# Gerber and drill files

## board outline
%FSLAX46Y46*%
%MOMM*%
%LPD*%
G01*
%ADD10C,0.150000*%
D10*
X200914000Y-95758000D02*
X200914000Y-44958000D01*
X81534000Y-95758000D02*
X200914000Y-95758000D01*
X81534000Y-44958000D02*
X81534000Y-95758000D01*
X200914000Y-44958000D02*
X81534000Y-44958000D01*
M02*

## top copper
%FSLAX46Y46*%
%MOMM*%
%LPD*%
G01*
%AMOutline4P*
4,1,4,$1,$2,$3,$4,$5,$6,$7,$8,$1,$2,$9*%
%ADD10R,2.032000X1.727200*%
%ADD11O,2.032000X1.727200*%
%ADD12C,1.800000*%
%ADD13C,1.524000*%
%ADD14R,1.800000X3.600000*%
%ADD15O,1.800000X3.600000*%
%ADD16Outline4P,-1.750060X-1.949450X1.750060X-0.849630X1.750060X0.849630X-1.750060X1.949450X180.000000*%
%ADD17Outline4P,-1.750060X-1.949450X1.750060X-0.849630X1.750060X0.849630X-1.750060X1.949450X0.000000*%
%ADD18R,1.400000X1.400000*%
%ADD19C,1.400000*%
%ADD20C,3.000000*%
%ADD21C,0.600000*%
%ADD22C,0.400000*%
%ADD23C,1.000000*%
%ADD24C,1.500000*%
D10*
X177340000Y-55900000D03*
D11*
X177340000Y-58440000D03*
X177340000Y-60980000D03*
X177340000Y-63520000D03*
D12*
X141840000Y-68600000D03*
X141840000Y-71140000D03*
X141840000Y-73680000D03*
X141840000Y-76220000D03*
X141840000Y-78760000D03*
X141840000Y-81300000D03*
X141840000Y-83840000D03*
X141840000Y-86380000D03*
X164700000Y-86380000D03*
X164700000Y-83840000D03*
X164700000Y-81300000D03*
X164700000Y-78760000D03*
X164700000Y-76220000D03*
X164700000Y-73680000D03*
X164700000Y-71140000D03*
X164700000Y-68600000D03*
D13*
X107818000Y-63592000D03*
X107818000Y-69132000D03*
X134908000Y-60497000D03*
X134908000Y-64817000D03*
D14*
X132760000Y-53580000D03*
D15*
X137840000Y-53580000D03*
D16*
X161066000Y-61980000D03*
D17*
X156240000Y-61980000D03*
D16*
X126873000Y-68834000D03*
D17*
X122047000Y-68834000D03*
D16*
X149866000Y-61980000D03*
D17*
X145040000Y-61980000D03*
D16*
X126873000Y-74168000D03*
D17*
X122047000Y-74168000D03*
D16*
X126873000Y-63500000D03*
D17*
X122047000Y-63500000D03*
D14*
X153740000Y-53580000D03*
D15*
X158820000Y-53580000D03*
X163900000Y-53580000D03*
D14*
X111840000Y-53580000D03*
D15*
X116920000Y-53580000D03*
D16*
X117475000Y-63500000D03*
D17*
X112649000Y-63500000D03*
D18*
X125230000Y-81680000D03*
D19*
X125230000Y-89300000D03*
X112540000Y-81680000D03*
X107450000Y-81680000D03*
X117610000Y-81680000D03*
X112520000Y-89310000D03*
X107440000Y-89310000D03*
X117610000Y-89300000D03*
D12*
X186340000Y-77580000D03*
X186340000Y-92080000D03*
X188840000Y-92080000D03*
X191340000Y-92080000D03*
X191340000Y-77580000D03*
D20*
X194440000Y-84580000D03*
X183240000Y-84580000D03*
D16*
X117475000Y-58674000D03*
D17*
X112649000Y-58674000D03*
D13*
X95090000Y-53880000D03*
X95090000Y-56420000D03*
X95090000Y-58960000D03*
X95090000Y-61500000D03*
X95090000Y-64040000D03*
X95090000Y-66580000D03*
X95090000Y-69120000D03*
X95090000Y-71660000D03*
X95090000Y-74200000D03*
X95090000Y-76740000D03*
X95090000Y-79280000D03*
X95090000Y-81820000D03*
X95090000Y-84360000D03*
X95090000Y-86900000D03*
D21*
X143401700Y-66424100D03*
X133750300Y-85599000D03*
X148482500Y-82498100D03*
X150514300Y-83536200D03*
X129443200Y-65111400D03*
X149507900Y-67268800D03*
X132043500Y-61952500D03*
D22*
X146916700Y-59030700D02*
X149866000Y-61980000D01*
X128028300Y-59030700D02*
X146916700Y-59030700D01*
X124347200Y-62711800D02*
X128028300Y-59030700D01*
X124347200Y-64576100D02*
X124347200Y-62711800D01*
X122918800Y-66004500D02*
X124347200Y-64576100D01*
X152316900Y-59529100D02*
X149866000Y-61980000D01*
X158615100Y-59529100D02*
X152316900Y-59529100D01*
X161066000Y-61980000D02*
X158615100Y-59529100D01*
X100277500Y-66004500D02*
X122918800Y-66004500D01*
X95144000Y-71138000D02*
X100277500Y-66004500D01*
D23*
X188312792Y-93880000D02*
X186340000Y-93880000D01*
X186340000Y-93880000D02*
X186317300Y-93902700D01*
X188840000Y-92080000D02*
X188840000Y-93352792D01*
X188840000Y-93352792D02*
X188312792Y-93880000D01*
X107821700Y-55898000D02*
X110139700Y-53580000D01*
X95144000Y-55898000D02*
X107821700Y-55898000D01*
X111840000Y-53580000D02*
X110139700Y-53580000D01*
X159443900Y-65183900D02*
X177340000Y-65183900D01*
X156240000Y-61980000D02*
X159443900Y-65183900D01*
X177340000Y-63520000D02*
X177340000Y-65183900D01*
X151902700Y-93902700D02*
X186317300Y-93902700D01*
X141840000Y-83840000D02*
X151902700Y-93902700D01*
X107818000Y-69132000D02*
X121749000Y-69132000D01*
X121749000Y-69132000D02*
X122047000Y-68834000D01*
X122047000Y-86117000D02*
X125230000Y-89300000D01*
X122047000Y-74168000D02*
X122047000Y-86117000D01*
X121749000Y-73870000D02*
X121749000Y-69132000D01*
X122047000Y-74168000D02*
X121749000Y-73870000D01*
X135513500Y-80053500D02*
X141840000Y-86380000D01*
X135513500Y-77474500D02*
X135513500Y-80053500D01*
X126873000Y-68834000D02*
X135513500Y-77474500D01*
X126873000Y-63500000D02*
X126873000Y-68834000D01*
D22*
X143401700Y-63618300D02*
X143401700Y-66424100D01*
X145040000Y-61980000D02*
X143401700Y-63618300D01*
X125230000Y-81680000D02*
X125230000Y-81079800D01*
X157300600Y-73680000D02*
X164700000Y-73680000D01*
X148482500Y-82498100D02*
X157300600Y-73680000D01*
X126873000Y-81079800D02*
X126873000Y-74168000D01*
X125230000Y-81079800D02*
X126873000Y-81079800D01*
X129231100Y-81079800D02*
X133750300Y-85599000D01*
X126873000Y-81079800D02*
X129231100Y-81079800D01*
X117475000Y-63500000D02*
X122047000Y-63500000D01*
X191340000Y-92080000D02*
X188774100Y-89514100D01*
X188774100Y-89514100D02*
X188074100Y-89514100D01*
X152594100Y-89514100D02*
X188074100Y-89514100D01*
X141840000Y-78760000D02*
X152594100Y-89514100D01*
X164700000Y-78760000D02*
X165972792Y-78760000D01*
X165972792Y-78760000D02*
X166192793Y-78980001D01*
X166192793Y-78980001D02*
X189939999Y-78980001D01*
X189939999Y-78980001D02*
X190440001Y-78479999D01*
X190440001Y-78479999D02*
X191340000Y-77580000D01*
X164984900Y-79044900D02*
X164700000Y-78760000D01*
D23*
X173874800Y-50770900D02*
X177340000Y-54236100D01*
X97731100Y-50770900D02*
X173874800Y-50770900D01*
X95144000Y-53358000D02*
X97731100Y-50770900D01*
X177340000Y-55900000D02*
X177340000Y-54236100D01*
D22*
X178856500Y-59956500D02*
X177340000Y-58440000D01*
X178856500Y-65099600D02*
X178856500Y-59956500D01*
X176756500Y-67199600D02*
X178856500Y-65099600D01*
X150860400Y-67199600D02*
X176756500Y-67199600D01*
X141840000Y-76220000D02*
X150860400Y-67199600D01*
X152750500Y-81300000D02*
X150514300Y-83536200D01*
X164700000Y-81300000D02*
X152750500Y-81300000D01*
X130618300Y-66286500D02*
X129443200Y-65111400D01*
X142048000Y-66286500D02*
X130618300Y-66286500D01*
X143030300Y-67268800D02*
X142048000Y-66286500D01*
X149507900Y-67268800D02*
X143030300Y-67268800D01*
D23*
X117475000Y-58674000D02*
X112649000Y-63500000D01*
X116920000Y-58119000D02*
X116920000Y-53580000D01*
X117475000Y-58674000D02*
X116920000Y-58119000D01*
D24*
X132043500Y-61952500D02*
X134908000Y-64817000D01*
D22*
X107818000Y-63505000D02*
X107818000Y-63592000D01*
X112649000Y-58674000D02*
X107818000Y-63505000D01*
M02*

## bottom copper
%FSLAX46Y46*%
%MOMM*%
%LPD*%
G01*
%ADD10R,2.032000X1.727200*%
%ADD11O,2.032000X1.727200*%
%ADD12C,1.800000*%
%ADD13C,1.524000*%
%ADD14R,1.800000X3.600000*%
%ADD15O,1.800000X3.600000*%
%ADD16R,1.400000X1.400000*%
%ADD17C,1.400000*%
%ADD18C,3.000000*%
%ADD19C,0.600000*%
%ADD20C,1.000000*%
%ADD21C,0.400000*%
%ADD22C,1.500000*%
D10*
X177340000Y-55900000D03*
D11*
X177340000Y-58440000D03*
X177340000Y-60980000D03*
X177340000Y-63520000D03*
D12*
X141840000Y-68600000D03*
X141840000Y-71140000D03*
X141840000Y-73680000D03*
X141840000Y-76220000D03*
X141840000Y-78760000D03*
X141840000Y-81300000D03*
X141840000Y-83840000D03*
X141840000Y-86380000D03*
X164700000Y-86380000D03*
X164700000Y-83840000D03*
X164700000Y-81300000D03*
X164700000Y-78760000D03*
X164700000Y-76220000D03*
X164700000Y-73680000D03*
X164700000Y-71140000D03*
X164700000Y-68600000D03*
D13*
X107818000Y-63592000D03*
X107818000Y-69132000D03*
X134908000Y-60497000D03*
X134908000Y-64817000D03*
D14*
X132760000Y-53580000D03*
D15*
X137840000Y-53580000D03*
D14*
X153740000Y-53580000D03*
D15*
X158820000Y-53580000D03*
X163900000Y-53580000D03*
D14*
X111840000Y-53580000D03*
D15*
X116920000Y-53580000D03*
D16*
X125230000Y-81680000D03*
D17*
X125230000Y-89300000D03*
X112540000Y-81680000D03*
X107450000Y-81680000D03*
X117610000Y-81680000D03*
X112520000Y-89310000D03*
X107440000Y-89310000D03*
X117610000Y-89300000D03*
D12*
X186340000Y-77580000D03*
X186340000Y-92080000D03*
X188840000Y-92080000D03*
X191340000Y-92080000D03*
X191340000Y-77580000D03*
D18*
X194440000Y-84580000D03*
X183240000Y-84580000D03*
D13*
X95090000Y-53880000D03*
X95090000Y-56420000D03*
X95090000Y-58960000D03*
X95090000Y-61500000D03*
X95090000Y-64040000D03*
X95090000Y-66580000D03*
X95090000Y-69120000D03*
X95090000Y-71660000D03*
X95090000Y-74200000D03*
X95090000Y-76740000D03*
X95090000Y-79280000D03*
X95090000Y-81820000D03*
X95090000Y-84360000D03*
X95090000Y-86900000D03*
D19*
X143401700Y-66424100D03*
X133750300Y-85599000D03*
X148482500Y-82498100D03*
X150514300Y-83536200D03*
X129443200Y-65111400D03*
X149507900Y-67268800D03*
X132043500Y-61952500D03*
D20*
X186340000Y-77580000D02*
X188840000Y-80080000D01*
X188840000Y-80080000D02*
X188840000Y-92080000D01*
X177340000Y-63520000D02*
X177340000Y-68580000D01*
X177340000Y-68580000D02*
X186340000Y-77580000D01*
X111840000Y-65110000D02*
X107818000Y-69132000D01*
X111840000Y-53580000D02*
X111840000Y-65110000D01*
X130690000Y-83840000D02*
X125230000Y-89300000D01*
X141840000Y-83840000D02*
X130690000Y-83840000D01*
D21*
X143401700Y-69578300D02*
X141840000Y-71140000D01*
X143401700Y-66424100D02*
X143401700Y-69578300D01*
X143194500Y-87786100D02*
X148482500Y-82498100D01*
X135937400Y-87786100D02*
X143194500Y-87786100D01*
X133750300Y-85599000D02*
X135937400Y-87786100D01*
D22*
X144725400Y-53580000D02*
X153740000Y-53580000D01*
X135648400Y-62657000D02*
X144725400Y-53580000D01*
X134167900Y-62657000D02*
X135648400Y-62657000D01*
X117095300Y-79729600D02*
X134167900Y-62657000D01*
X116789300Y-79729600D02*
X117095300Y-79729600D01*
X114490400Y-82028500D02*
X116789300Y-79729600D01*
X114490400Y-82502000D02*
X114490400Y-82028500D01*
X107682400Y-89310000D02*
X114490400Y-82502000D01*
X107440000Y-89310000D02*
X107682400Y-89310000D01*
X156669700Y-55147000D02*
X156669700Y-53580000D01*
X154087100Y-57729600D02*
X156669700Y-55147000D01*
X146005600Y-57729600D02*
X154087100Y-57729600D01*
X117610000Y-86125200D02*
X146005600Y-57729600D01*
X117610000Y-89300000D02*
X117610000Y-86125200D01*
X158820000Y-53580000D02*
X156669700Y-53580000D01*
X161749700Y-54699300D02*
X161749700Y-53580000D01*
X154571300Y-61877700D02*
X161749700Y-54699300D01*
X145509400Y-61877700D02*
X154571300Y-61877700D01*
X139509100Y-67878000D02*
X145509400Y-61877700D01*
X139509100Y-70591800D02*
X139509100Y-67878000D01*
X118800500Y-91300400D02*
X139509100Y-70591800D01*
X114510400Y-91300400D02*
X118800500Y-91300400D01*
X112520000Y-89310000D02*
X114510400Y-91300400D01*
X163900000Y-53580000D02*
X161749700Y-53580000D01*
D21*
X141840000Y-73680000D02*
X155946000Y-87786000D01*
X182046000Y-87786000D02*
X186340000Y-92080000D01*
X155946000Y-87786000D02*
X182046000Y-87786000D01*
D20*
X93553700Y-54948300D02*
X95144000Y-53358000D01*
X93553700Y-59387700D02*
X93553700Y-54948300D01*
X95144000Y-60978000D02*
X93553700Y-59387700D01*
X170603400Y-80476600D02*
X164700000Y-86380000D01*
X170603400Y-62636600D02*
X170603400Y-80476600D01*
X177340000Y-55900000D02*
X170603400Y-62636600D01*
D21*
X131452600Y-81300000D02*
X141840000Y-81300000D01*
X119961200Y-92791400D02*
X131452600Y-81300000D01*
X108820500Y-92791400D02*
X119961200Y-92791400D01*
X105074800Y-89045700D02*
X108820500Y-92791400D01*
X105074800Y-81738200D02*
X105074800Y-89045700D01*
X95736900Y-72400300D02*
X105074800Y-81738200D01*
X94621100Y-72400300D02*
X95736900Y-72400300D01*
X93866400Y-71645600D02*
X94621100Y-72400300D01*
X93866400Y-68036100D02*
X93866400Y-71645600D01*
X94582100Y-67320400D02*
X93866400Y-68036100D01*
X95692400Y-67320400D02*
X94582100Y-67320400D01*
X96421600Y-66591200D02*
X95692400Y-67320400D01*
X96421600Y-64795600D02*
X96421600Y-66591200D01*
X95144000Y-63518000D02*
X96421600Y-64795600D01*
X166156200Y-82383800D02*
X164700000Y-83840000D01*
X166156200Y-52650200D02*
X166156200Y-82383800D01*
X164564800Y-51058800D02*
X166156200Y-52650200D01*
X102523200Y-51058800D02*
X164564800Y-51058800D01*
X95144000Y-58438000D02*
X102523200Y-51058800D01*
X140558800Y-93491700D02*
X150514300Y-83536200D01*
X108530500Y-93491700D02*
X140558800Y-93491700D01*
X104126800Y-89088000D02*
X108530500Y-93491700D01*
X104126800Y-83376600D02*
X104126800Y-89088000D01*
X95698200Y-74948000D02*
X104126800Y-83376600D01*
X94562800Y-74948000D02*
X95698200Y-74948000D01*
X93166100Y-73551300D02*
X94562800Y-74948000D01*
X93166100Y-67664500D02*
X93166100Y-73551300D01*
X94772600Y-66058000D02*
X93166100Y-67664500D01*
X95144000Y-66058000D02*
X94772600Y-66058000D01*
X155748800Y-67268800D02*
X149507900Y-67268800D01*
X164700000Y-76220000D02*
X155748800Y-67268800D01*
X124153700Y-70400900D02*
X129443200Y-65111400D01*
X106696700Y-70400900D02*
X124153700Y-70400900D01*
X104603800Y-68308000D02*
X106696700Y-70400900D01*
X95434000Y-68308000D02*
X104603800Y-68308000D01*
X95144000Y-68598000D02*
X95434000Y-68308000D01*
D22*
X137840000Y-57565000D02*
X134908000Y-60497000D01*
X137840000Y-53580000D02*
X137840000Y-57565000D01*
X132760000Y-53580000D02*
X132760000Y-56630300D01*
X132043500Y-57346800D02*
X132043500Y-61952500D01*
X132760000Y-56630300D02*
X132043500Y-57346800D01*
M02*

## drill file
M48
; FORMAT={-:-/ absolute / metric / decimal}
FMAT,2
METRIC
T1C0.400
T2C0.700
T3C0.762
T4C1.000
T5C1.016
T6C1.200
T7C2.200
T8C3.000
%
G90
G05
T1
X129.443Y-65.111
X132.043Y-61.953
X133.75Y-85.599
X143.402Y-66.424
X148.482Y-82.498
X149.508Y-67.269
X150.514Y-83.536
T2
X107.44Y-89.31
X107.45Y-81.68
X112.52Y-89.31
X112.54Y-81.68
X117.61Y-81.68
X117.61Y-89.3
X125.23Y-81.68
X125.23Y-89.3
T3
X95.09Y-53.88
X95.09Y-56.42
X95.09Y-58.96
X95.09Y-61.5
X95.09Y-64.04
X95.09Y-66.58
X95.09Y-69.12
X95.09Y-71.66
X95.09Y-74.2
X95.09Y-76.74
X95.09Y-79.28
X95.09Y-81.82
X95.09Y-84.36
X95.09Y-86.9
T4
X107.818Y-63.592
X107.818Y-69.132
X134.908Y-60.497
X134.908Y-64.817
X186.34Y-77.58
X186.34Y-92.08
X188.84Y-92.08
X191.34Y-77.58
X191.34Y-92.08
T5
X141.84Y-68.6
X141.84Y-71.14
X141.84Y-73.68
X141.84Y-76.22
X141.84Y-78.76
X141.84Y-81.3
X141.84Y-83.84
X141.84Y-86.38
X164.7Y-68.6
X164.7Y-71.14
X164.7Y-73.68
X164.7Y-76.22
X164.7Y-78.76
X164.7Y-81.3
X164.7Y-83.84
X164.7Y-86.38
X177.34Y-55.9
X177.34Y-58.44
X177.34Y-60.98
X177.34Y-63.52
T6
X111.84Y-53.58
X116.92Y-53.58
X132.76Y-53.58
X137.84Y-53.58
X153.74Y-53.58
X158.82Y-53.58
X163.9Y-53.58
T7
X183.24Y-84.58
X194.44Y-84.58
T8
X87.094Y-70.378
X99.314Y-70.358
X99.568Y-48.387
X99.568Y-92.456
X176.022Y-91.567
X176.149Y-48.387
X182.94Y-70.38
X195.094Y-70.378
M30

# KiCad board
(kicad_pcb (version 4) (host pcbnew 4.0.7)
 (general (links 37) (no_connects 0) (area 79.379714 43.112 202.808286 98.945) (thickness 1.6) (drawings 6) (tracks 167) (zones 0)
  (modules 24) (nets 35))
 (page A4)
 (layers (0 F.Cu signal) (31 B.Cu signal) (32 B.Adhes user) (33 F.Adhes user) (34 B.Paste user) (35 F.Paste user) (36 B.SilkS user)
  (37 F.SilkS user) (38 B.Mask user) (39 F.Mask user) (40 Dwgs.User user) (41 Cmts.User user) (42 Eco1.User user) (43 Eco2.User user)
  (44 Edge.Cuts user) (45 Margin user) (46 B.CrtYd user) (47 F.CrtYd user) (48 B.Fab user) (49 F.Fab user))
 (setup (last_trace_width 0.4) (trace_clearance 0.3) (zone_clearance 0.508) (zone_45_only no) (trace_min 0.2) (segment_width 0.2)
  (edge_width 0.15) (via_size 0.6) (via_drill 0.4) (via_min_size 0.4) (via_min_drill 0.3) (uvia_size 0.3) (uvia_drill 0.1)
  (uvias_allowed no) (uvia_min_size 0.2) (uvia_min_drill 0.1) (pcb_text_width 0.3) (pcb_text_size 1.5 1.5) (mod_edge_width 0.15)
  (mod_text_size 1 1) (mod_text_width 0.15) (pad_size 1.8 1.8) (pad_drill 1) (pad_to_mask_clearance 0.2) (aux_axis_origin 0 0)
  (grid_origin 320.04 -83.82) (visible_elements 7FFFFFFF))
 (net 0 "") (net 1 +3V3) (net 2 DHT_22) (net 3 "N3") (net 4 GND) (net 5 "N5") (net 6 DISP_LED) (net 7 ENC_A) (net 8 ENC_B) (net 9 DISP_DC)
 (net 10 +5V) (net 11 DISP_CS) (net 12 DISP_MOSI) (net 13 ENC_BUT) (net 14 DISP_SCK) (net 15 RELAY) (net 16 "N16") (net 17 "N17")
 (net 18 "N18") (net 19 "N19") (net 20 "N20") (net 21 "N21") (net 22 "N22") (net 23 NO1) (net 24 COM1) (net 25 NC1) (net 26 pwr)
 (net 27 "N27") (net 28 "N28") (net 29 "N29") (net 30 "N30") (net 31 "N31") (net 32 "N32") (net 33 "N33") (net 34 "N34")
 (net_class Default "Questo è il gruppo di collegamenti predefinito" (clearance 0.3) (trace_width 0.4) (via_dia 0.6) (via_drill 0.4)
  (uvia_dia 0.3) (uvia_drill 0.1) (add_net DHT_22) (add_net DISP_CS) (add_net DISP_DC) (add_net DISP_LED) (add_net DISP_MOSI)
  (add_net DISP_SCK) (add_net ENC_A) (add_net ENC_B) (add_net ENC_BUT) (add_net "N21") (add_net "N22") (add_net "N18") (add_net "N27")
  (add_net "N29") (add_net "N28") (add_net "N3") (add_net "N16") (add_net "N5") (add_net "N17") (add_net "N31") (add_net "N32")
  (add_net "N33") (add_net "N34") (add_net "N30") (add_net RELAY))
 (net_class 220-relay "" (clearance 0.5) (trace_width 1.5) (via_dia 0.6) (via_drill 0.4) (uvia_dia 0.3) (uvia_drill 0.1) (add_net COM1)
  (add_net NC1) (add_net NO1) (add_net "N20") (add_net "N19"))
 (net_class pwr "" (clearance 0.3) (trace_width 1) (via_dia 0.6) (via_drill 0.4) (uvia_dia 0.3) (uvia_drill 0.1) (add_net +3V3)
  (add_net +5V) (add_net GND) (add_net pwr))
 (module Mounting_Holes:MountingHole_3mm (layer F.Cu) (at 182.94 70.38 180)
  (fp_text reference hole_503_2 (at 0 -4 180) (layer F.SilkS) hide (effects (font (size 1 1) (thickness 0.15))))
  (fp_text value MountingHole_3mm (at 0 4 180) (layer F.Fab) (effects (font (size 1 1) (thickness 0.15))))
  (pad 1 np_thru_hole circle (at 0 0 180) (size 3 3) (drill 3) (layers *.Cu *.Mask)))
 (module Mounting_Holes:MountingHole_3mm (layer F.Cu) (at 176.149 48.387 180)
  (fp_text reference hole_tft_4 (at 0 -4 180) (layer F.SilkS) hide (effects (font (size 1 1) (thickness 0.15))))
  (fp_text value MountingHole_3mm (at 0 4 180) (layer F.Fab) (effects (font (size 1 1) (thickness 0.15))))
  (pad 1 np_thru_hole circle (at 0 0 180) (size 3 3) (drill 3) (layers *.Cu *.Mask)))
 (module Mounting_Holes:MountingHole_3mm (layer F.Cu) (at 99.568 48.387 180)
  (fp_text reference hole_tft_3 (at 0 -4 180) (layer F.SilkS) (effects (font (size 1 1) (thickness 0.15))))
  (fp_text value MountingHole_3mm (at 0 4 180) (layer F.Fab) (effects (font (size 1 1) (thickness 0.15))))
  (pad 1 np_thru_hole circle (at 0 0 180) (size 3 3) (drill 3) (layers *.Cu *.Mask)))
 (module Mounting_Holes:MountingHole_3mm (layer F.Cu) (at 99.568 92.456 180)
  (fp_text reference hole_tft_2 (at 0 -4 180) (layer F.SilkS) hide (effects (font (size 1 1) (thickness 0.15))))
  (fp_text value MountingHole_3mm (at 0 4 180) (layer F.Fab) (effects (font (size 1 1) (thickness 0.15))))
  (pad 1 np_thru_hole circle (at 0 0 180) (size 3 3) (drill 3) (layers *.Cu *.Mask)))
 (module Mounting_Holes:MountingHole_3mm (layer F.Cu) (at 87.094 70.378 180)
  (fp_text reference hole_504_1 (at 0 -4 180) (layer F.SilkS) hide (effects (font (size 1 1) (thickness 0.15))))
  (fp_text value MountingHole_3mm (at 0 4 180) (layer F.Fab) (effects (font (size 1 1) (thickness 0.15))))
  (pad 1 np_thru_hole circle (at 0 0 180) (size 3 3) (drill 3) (layers *.Cu *.Mask)))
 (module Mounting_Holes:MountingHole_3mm (layer F.Cu) (at 195.094 70.378 180)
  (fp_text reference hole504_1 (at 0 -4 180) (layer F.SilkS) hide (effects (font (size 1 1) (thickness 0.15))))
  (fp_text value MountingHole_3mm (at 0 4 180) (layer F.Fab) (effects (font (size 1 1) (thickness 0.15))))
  (pad 1 np_thru_hole circle (at 0 0 180) (size 3 3) (drill 3) (layers *.Cu *.Mask)))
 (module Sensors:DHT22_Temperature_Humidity (layer F.Cu) (at 177.34 59.71 270)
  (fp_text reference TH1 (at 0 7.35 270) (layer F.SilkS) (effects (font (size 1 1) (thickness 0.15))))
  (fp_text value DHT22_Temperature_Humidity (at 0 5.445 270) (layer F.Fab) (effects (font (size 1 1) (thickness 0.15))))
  (pad 1 thru_hole rect (at -3.81 0) (size 2.032 1.7272) (drill 1.016) (layers *.Cu *.Mask F.SilkS) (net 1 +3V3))
  (pad 2 thru_hole oval (at -1.27 0) (size 2.032 1.7272) (drill 1.016) (layers *.Cu *.Mask F.SilkS) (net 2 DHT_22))
  (pad 3 thru_hole oval (at 1.27 0) (size 2.032 1.7272) (drill 1.016) (layers *.Cu *.Mask F.SilkS) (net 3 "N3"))
  (pad 4 thru_hole oval (at 3.81 0) (size 2.032 1.7272) (drill 1.016) (layers *.Cu *.Mask F.SilkS) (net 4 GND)))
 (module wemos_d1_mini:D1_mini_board (layer F.Cu) (at 153.27 78.76)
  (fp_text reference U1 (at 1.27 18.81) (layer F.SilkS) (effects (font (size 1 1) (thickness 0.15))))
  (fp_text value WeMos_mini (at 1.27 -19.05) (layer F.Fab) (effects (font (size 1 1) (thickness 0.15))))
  (pad 8 thru_hole circle (at -11.43 -10.16) (size 1.8 1.8) (drill 1.016) (layers *.Cu *.Mask F.SilkS) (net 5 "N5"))
  (pad 7 thru_hole circle (at -11.43 -7.62) (size 1.8 1.8) (drill 1.016) (layers *.Cu *.Mask F.SilkS) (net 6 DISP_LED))
  (pad 6 thru_hole circle (at -11.43 -5.08) (size 1.8 1.8) (drill 1.016) (layers *.Cu *.Mask F.SilkS) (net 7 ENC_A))
  (pad 5 thru_hole circle (at -11.43 -2.54) (size 1.8 1.8) (drill 1.016) (layers *.Cu *.Mask F.SilkS) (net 2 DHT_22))
  (pad 4 thru_hole circle (at -11.43 0) (size 1.8 1.8) (drill 1.016) (layers *.Cu *.Mask F.SilkS) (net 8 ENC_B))
  (pad 3 thru_hole circle (at -11.43 2.54) (size 1.8 1.8) (drill 1.016) (layers *.Cu *.Mask F.SilkS) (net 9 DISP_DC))
  (pad 2 thru_hole circle (at -11.43 5.08) (size 1.8 1.8) (drill 1.016) (layers *.Cu *.Mask F.SilkS) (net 4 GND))
  (pad 1 thru_hole circle (at -11.43 7.62) (size 1.8 1.8) (drill 1.016) (layers *.Cu *.Mask F.SilkS) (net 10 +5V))
  (pad 16 thru_hole circle (at 11.43 7.62) (size 1.8 1.8) (drill 1.016) (layers *.Cu *.Mask F.SilkS) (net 1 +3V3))
  (pad 15 thru_hole circle (at 11.43 5.08) (size 1.8 1.8) (drill 1.016) (layers *.Cu *.Mask F.SilkS) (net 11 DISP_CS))
  (pad 14 thru_hole circle (at 11.43 2.54) (size 1.8 1.8) (drill 1.016) (layers *.Cu *.Mask F.SilkS) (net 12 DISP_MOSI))
  (pad 13 thru_hole circle (at 11.43 0) (size 1.8 1.8) (drill 1.016) (layers *.Cu *.Mask F.SilkS) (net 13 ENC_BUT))
  (pad 12 thru_hole circle (at 11.43 -2.54) (size 1.8 1.8) (drill 1.016) (layers *.Cu *.Mask F.SilkS) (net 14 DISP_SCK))
  (pad 11 thru_hole circle (at 11.43 -5.08) (size 1.8 1.8) (drill 1.016) (layers *.Cu *.Mask F.SilkS) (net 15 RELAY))
  (pad 10 thru_hole circle (at 11.43 -7.62) (size 1.8 1.8) (drill 1.016) (layers *.Cu *.Mask F.SilkS) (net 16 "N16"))
  (pad 9 thru_hole circle (at 11.43 -10.16) (size 1.8 1.8) (drill 1.016) (layers *.Cu *.Mask F.SilkS) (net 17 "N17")))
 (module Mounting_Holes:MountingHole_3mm (layer F.Cu) (at 99.314 70.358 180)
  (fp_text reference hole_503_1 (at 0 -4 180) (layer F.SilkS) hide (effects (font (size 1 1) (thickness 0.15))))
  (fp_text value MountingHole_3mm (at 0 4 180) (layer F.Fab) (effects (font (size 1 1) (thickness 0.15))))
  (pad 1 np_thru_hole circle (at 0 0 180) (size 3 3) (drill 3) (layers *.Cu *.Mask)))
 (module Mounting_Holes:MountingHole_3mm (layer F.Cu) (at 176.022 91.567 180) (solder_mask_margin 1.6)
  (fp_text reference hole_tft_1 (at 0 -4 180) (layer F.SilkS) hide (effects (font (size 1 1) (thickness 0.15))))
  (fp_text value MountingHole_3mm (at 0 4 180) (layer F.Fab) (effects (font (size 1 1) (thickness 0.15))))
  (pad 1 np_thru_hole circle (at 0 0 180) (size 3 3) (drill 3) (layers *.Cu *.Mask)))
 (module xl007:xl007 (layer F.Cu) (at 121.158 66.802)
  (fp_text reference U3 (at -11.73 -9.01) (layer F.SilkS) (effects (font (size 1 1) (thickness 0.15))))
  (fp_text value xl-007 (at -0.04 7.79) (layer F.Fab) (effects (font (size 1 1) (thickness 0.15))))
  (pad 3 thru_hole circle (at -13.34 -3.21) (size 1.524 1.524) (drill 1) (layers *.Cu *.Mask) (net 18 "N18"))
  (pad 4 thru_hole circle (at -13.34 2.33) (size 1.524 1.524) (drill 1) (layers *.Cu *.Mask) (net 4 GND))
  (pad 1 thru_hole circle (at 13.75 -6.305) (size 1.524 1.524) (drill 1) (layers *.Cu *.Mask) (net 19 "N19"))
  (pad 2 thru_hole circle (at 13.75 -1.985) (size 1.524 1.524) (drill 1) (layers *.Cu *.Mask) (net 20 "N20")))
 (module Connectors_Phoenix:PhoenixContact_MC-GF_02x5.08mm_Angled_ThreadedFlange (layer B.Cu) (at 132.76 53.58)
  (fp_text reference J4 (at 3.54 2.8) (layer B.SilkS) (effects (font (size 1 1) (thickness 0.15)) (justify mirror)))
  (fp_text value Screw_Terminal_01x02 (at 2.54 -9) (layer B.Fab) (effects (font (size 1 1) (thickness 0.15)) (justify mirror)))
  (pad 1 thru_hole rect (at 0 0) (size 1.8 3.6) (drill 1.2) (layers *.Cu *.Mask) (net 20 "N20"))
  (pad 2 thru_hole oval (at 5.08 0) (size 1.8 3.6) (drill 1.2) (layers *.Cu *.Mask) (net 19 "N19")))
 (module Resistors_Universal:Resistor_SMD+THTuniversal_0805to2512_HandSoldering (layer F.Cu) (at 158.653 61.98 180)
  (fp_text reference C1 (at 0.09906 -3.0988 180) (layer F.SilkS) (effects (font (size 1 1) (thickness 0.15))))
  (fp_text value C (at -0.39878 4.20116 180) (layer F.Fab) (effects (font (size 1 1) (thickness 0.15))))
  (pad 1 smd trapezoid (at -2.413 0 180) (size 3.50012 2.79908) (rect_delta 1.09982 0) (layers F.Cu F.Paste F.Mask) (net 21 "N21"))
  (pad 2 smd trapezoid (at 2.413 0) (size 3.50012 2.79908) (rect_delta 1.09982 0) (layers F.Cu F.Paste F.Mask) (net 4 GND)))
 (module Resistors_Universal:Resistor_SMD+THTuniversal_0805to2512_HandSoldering (layer F.Cu) (at 124.46 68.834 180)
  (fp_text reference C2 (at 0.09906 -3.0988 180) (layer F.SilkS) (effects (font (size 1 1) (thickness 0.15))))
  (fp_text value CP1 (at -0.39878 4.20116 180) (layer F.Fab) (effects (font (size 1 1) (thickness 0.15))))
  (pad 1 smd trapezoid (at -2.413 0 180) (size 3.50012 2.79908) (rect_delta 1.09982 0) (layers F.Cu F.Paste F.Mask) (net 10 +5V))
  (pad 2 smd trapezoid (at 2.413 0) (size 3.50012 2.79908) (rect_delta 1.09982 0) (layers F.Cu F.Paste F.Mask) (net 4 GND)))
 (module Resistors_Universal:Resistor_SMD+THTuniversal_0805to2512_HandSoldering (layer F.Cu) (at 147.453 61.98 180)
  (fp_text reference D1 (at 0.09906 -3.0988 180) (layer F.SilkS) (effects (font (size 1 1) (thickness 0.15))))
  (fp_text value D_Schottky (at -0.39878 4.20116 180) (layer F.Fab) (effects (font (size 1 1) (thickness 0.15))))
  (pad 1 smd trapezoid (at -2.413 0 180) (size 3.50012 2.79908) (rect_delta 1.09982 0) (layers F.Cu F.Paste F.Mask) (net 21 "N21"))
  (pad 2 smd trapezoid (at 2.413 0) (size 3.50012 2.79908) (rect_delta 1.09982 0) (layers F.Cu F.Paste F.Mask) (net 6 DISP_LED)))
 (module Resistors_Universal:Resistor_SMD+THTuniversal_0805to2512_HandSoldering (layer F.Cu) (at 124.46 74.168 180)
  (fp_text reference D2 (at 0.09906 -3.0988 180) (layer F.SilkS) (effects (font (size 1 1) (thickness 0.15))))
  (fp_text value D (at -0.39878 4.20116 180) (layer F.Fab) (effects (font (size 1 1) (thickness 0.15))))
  (pad 1 smd trapezoid (at -2.413 0 180) (size 3.50012 2.79908) (rect_delta 1.09982 0) (layers F.Cu F.Paste F.Mask) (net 15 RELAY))
  (pad 2 smd trapezoid (at 2.413 0) (size 3.50012 2.79908) (rect_delta 1.09982 0) (layers F.Cu F.Paste F.Mask) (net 4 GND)))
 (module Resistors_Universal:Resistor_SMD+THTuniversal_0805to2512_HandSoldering (layer F.Cu) (at 124.46 63.5 180)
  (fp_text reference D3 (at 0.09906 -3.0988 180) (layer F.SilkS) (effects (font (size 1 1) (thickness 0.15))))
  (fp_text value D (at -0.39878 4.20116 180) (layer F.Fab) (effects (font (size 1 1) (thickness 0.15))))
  (pad 1 smd trapezoid (at -2.413 0 180) (size 3.50012 2.79908) (rect_delta 1.09982 0) (layers F.Cu F.Paste F.Mask) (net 10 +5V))
  (pad 2 smd trapezoid (at 2.413 0) (size 3.50012 2.79908) (rect_delta 1.09982 0) (layers F.Cu F.Paste F.Mask) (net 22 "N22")))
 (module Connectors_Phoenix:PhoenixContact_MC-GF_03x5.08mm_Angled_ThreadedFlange (layer B.Cu) (at 153.74 53.58)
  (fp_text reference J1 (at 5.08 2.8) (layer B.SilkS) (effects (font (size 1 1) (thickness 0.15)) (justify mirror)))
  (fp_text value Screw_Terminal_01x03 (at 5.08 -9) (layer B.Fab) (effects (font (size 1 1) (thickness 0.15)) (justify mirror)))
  (pad 1 thru_hole rect (at 0 0) (size 1.8 3.6) (drill 1.2) (layers *.Cu *.Mask) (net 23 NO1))
  (pad 2 thru_hole oval (at 5.08 0) (size 1.8 3.6) (drill 1.2) (layers *.Cu *.Mask) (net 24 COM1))
  (pad 3 thru_hole oval (at 10.16 0) (size 1.8 3.6) (drill 1.2) (layers *.Cu *.Mask) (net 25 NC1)))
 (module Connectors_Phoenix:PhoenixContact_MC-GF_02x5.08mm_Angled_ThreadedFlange (layer B.Cu) (at 111.84 53.58)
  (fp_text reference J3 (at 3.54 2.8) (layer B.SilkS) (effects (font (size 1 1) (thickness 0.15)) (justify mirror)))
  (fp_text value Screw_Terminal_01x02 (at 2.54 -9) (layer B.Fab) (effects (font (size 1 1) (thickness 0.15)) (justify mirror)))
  (pad 1 thru_hole rect (at 0 0) (size 1.8 3.6) (drill 1.2) (layers *.Cu *.Mask) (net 4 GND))
  (pad 2 thru_hole oval (at 5.08 0) (size 1.8 3.6) (drill 1.2) (layers *.Cu *.Mask) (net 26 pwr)))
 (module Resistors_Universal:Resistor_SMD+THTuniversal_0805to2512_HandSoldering (layer F.Cu) (at 115.062 63.5 180)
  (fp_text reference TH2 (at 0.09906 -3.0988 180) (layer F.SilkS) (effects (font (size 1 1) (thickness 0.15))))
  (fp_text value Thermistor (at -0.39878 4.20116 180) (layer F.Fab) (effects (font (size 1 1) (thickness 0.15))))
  (pad 1 smd trapezoid (at -2.413 0 180) (size 3.50012 2.79908) (rect_delta 1.09982 0) (layers F.Cu F.Paste F.Mask) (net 22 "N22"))
  (pad 2 smd trapezoid (at 2.413 0) (size 3.50012 2.79908) (rect_delta 1.09982 0) (layers F.Cu F.Paste F.Mask) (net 26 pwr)))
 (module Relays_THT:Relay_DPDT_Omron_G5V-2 (layer F.Cu) (at 125.23 81.68 270)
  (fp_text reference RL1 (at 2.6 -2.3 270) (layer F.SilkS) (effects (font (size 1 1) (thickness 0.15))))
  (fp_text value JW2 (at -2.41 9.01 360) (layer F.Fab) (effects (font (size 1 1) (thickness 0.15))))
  (pad 1 thru_hole rect (at 0 0 270) (size 1.4 1.4) (drill 0.7) (layers *.Cu *.Mask) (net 15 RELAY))
  (pad 8 thru_hole circle (at 7.62 0 270) (size 1.4 1.4) (drill 0.7) (layers *.Cu *.Mask) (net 4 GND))
  (pad 2 thru_hole circle (at 0 12.69 270) (size 1.4 1.4) (drill 0.7) (layers *.Cu *.Mask) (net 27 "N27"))
  (pad 4 thru_hole circle (at 0 17.78 270) (size 1.4 1.4) (drill 0.7) (layers *.Cu *.Mask) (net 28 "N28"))
  (pad 3 thru_hole circle (at 0 7.62 270) (size 1.4 1.4) (drill 0.7) (layers *.Cu *.Mask) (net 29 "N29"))
  (pad 7 thru_hole circle (at 7.63 12.71 270) (size 1.4 1.4) (drill 0.7) (layers *.Cu *.Mask) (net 25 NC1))
  (pad 5 thru_hole circle (at 7.63 17.79 270) (size 1.4 1.4) (drill 0.7) (layers *.Cu *.Mask) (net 23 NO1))
  (pad 6 thru_hole circle (at 7.62 7.62 270) (size 1.4 1.4) (drill 0.7) (layers *.Cu *.Mask) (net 24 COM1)))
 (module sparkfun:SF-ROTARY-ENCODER (layer F.Cu) (at 188.84 84.58)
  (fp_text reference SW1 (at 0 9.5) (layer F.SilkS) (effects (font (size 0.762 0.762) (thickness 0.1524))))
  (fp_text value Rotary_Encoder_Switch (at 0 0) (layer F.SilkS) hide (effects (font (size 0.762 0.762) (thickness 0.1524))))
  (pad 5 thru_hole circle (at -2.5 -7) (size 1.8 1.8) (drill 1) (layers *.Cu *.Mask F.SilkS) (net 4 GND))
  (pad 1 thru_hole circle (at -2.5 7.5) (size 1.8 1.8) (drill 1) (layers *.Cu *.Mask F.SilkS) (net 7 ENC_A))
  (pad 2 thru_hole circle (at 0 7.5) (size 1.8 1.8) (drill 1) (layers *.Cu *.Mask F.SilkS) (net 4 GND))
  (pad 3 thru_hole circle (at 2.5 7.5) (size 1.8 1.8) (drill 1) (layers *.Cu *.Mask F.SilkS) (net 8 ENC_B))
  (pad 4 thru_hole circle (at 2.5 -7) (size 1.8 1.8) (drill 1) (layers *.Cu *.Mask F.SilkS) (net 13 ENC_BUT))
  (pad "" thru_hole circle (at 5.6 0) (size 3 3) (drill 2.2) (layers *.Cu *.Mask F.SilkS))
  (pad "" thru_hole circle (at -5.6 0) (size 3 3) (drill 2.2) (layers *.Cu *.Mask F.SilkS)))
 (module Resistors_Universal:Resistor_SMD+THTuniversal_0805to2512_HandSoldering (layer F.Cu) (at 115.062 58.674 180)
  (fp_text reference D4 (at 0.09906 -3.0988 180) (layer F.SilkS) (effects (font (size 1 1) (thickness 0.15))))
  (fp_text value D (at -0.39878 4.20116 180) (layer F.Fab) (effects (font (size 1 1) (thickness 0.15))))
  (pad 1 smd trapezoid (at -2.413 0 180) (size 3.50012 2.79908) (rect_delta 1.09982 0) (layers F.Cu F.Paste F.Mask) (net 26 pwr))
  (pad 2 smd trapezoid (at 2.413 0) (size 3.50012 2.79908) (rect_delta 1.09982 0) (layers F.Cu F.Paste F.Mask) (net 18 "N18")))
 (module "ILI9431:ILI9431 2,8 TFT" (layer F.Cu) (at 136.09 70.38)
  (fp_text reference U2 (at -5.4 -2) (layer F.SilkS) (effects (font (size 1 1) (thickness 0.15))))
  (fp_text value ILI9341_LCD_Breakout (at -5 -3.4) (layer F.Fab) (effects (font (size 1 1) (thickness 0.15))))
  (pad 1 thru_hole circle (at -41 -16.5) (size 1.524 1.524) (drill 0.762) (layers *.Cu *.Mask) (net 1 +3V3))
  (pad 2 thru_hole circle (at -41 -13.96) (size 1.524 1.524) (drill 0.762) (layers *.Cu *.Mask) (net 4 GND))
  (pad 3 thru_hole circle (at -41 -11.42) (size 1.524 1.524) (drill 0.762) (layers *.Cu *.Mask) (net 11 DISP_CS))
  (pad 4 thru_hole circle (at -41 -8.88) (size 1.524 1.524) (drill 0.762) (layers *.Cu *.Mask) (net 1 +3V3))
  (pad 5 thru_hole circle (at -41 -6.34) (size 1.524 1.524) (drill 0.762) (layers *.Cu *.Mask) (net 9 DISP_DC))
  (pad 6 thru_hole circle (at -41 -3.8) (size 1.524 1.524) (drill 0.762) (layers *.Cu *.Mask) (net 12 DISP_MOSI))
  (pad 7 thru_hole circle (at -41 -1.26) (size 1.524 1.524) (drill 0.762) (layers *.Cu *.Mask) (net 14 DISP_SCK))
  (pad 8 thru_hole circle (at -41 1.28) (size 1.524 1.524) (drill 0.762) (layers *.Cu *.Mask) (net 21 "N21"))
  (pad 9 thru_hole circle (at -41 3.82) (size 1.524 1.524) (drill 0.762) (layers *.Cu *.Mask) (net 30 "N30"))
  (pad 10 thru_hole circle (at -41 6.36) (size 1.524 1.524) (drill 0.762) (layers *.Cu *.Mask) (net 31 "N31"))
  (pad 11 thru_hole circle (at -41 8.9) (size 1.524 1.524) (drill 0.762) (layers *.Cu *.Mask) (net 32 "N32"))
  (pad 12 thru_hole circle (at -41 11.44) (size 1.524 1.524) (drill 0.762) (layers *.Cu *.Mask) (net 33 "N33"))
  (pad 13 thru_hole circle (at -41 13.98) (size 1.524 1.524) (drill 0.762) (layers *.Cu *.Mask) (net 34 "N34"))
  (pad 14 thru_hole circle (at -41 16.52) (size 1.524 1.524) (drill 0.762) (layers *.Cu *.Mask)))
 (gr_line (start 200.914 95.758) (end 200.914 44.958) (layer Edge.Cuts) (width 0.15))
 (gr_line (start 81.534 95.758) (end 200.914 95.758) (layer Edge.Cuts) (width 0.15))
 (gr_line (start 81.534 44.958) (end 81.534 95.758) (layer Edge.Cuts) (width 0.15))
 (gr_line (start 200.914 44.958) (end 81.534 44.958) (layer Edge.Cuts) (width 0.15))
 (segment (start 146.9167 59.0307) (end 149.866 61.98) (width 0.4) (layer F.Cu) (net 21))
 (segment (start 128.0283 59.0307) (end 146.9167 59.0307) (width 0.4) (layer F.Cu) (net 21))
 (segment (start 124.3472 62.7118) (end 128.0283 59.0307) (width 0.4) (layer F.Cu) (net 21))
 (segment (start 124.3472 64.5761) (end 124.3472 62.7118) (width 0.4) (layer F.Cu) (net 21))
 (segment (start 122.9188 66.0045) (end 124.3472 64.5761) (width 0.4) (layer F.Cu) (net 21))
 (segment (start 152.3169 59.5291) (end 149.866 61.98) (width 0.4) (layer F.Cu) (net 21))
 (segment (start 158.6151 59.5291) (end 152.3169 59.5291) (width 0.4) (layer F.Cu) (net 21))
 (segment (start 161.066 61.98) (end 158.6151 59.5291) (width 0.4) (layer F.Cu) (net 21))
 (segment (start 100.2775 66.0045) (end 122.9188 66.0045) (width 0.4) (layer F.Cu) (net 21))
 (segment (start 95.144 71.138) (end 100.2775 66.0045) (width 0.4) (layer F.Cu) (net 21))
 (segment (start 188.312792 93.88) (end 186.34 93.88) (width 1) (layer F.Cu) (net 4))
 (segment (start 186.34 93.88) (end 186.3173 93.9027) (width 1) (layer F.Cu) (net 4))
 (segment (start 188.84 92.08) (end 188.84 93.352792) (width 1) (layer F.Cu) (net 4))
 (segment (start 188.84 93.352792) (end 188.312792 93.88) (width 1) (layer F.Cu) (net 4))
 (segment (start 186.34 77.58) (end 188.84 80.08) (width 1) (layer B.Cu) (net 4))
 (segment (start 188.84 80.08) (end 188.84 92.08) (width 1) (layer B.Cu) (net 4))
 (segment (start 177.34 63.52) (end 177.34 68.58) (width 1) (layer B.Cu) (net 4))
 (segment (start 177.34 68.58) (end 186.34 77.58) (width 1) (layer B.Cu) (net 4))
 (segment (start 107.8217 55.898) (end 110.1397 53.58) (width 1) (layer F.Cu) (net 4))
 (segment (start 95.144 55.898) (end 107.8217 55.898) (width 1) (layer F.Cu) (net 4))
 (segment (start 111.84 53.58) (end 110.1397 53.58) (width 1) (layer F.Cu) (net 4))
 (segment (start 159.4439 65.1839) (end 177.34 65.1839) (width 1) (layer F.Cu) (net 4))
 (segment (start 156.24 61.98) (end 159.4439 65.1839) (width 1) (layer F.Cu) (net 4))
 (segment (start 177.34 63.52) (end 177.34 65.1839) (width 1) (layer F.Cu) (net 4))
 (segment (start 111.84 65.11) (end 107.818 69.132) (width 1) (layer B.Cu) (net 4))
 (segment (start 111.84 53.58) (end 111.84 65.11) (width 1) (layer B.Cu) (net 4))
 (segment (start 151.9027 93.9027) (end 186.3173 93.9027) (width 1) (layer F.Cu) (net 4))
 (segment (start 141.84 83.84) (end 151.9027 93.9027) (width 1) (layer F.Cu) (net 4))
 (segment (start 130.69 83.84) (end 125.23 89.3) (width 1) (layer B.Cu) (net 4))
 (segment (start 141.84 83.84) (end 130.69 83.84) (width 1) (layer B.Cu) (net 4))
 (segment (start 107.818 69.132) (end 121.749 69.132) (width 1) (layer F.Cu) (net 4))
 (segment (start 121.749 69.132) (end 122.047 68.834) (width 1) (layer F.Cu) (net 4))
 (segment (start 122.047 86.117) (end 125.23 89.3) (width 1) (layer F.Cu) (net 4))
 (segment (start 122.047 74.168) (end 122.047 86.117) (width 1) (layer F.Cu) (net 4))
 (segment (start 121.749 73.87) (end 121.749 69.132) (width 1) (layer F.Cu) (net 4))
 (segment (start 122.047 74.168) (end 121.749 73.87) (width 1) (layer F.Cu) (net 4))
 (segment (start 135.5135 80.0535) (end 141.84 86.38) (width 1) (layer F.Cu) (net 10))
 (segment (start 135.5135 77.4745) (end 135.5135 80.0535) (width 1) (layer F.Cu) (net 10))
 (segment (start 126.873 68.834) (end 135.5135 77.4745) (width 1) (layer F.Cu) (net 10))
 (segment (start 126.873 63.5) (end 126.873 68.834) (width 1) (layer F.Cu) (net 10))
 (via (at 143.4017 66.4241) (size 0.6) (layers F.Cu B.Cu) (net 6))
 (segment (start 143.4017 63.6183) (end 143.4017 66.4241) (width 0.4) (layer F.Cu) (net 6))
 (segment (start 145.04 61.98) (end 143.4017 63.6183) (width 0.4) (layer F.Cu) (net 6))
 (segment (start 143.4017 69.5783) (end 141.84 71.14) (width 0.4) (layer B.Cu) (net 6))
 (segment (start 143.4017 66.4241) (end 143.4017 69.5783) (width 0.4) (layer B.Cu) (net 6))
 (via (at 133.7503 85.599) (size 0.6) (layers F.Cu B.Cu) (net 15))
 (via (at 148.4825 82.4981) (size 0.6) (layers F.Cu B.Cu) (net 15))
 (segment (start 125.23 81.68) (end 125.23 81.0798) (width 0.4) (layer F.Cu) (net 15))
 (segment (start 143.1945 87.7861) (end 148.4825 82.4981) (width 0.4) (layer B.Cu) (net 15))
 (segment (start 135.9374 87.7861) (end 143.1945 87.7861) (width 0.4) (layer B.Cu) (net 15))
 (segment (start 133.7503 85.599) (end 135.9374 87.7861) (width 0.4) (layer B.Cu) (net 15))
 (segment (start 157.3006 73.68) (end 164.7 73.68) (width 0.4) (layer F.Cu) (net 15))
 (segment (start 148.4825 82.4981) (end 157.3006 73.68) (width 0.4) (layer F.Cu) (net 15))
 (segment (start 126.873 81.0798) (end 126.873 74.168) (width 0.4) (layer F.Cu) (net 15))
 (segment (start 125.23 81.0798) (end 126.873 81.0798) (width 0.4) (layer F.Cu) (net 15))
 (segment (start 129.2311 81.0798) (end 133.7503 85.599) (width 0.4) (layer F.Cu) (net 15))
 (segment (start 126.873 81.0798) (end 129.2311 81.0798) (width 0.4) (layer F.Cu) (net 15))
 (segment (start 117.475 63.5) (end 122.047 63.5) (width 0.4) (layer F.Cu) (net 22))
 (segment (start 144.7254 53.58) (end 153.74 53.58) (width 1.5) (layer B.Cu) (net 23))
 (segment (start 135.6484 62.657) (end 144.7254 53.58) (width 1.5) (layer B.Cu) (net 23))
 (segment (start 134.1679 62.657) (end 135.6484 62.657) (width 1.5) (layer B.Cu) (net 23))
 (segment (start 117.0953 79.7296) (end 134.1679 62.657) (width 1.5) (layer B.Cu) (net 23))
 (segment (start 116.7893 79.7296) (end 117.0953 79.7296) (width 1.5) (layer B.Cu) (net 23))
 (segment (start 114.4904 82.0285) (end 116.7893 79.7296) (width 1.5) (layer B.Cu) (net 23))
 (segment (start 114.4904 82.502) (end 114.4904 82.0285) (width 1.5) (layer B.Cu) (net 23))
 (segment (start 107.6824 89.31) (end 114.4904 82.502) (width 1.5) (layer B.Cu) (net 23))
 (segment (start 107.44 89.31) (end 107.6824 89.31) (width 1.5) (layer B.Cu) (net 23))
 (segment (start 156.6697 55.147) (end 156.6697 53.58) (width 1.5) (layer B.Cu) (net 24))
 (segment (start 154.0871 57.7296) (end 156.6697 55.147) (width 1.5) (layer B.Cu) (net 24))
 (segment (start 146.0056 57.7296) (end 154.0871 57.7296) (width 1.5) (layer B.Cu) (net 24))
 (segment (start 117.61 86.1252) (end 146.0056 57.7296) (width 1.5) (layer B.Cu) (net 24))
 (segment (start 117.61 89.3) (end 117.61 86.1252) (width 1.5) (layer B.Cu) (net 24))
 (segment (start 158.82 53.58) (end 156.6697 53.58) (width 1.5) (layer B.Cu) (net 24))
 (segment (start 161.7497 54.6993) (end 161.7497 53.58) (width 1.5) (layer B.Cu) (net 25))
 (segment (start 154.5713 61.8777) (end 161.7497 54.6993) (width 1.5) (layer B.Cu) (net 25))
 (segment (start 145.5094 61.8777) (end 154.5713 61.8777) (width 1.5) (layer B.Cu) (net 25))
 (segment (start 139.5091 67.878) (end 145.5094 61.8777) (width 1.5) (layer B.Cu) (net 25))
 (segment (start 139.5091 70.5918) (end 139.5091 67.878) (width 1.5) (layer B.Cu) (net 25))
 (segment (start 118.8005 91.3004) (end 139.5091 70.5918) (width 1.5) (layer B.Cu) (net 25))
 (segment (start 114.5104 91.3004) (end 118.8005 91.3004) (width 1.5) (layer B.Cu) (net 25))
 (segment (start 112.52 89.31) (end 114.5104 91.3004) (width 1.5) (layer B.Cu) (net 25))
 (segment (start 163.9 53.58) (end 161.7497 53.58) (width 1.5) (layer B.Cu) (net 25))
 (segment (start 141.84 73.68) (end 155.946 87.786) (width 0.4) (layer B.Cu) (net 7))
 (segment (start 182.046 87.786) (end 186.34 92.08) (width 0.4) (layer B.Cu) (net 7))
 (segment (start 155.946 87.786) (end 182.046 87.786) (width 0.4) (layer B.Cu) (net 7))
 (segment (start 191.34 92.08) (end 188.7741 89.5141) (width 0.4) (layer F.Cu) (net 8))
 (segment (start 188.7741 89.5141) (end 188.0741 89.5141) (width 0.4) (layer F.Cu) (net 8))
 (segment (start 152.5941 89.5141) (end 188.0741 89.5141) (width 0.4) (layer F.Cu) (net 8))
 (segment (start 141.84 78.76) (end 152.5941 89.5141) (width 0.4) (layer F.Cu) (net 8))
 (segment (start 164.7 78.76) (end 165.972792 78.76) (width 0.4) (layer F.Cu) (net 13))
 (segment (start 165.972792 78.76) (end 166.192793 78.980001) (width 0.4) (layer F.Cu) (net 13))
 (segment (start 166.192793 78.980001) (end 189.939999 78.980001) (width 0.4) (layer F.Cu) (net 13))
 (segment (start 189.939999 78.980001) (end 190.440001 78.479999) (width 0.4) (layer F.Cu) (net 13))
 (segment (start 190.440001 78.479999) (end 191.34 77.58) (width 0.4) (layer F.Cu) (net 13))
 (segment (start 164.9849 79.0449) (end 164.7 78.76) (width 0.4) (layer F.Cu) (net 13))
 (segment (start 93.5537 54.9483) (end 95.144 53.358) (width 1) (layer B.Cu) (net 1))
 (segment (start 93.5537 59.3877) (end 93.5537 54.9483) (width 1) (layer B.Cu) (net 1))
 (segment (start 95.144 60.978) (end 93.5537 59.3877) (width 1) (layer B.Cu) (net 1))
 (segment (start 173.8748 50.7709) (end 177.34 54.2361) (width 1) (layer F.Cu) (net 1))
 (segment (start 97.7311 50.7709) (end 173.8748 50.7709) (width 1) (layer F.Cu) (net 1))
 (segment (start 95.144 53.358) (end 97.7311 50.7709) (width 1) (layer F.Cu) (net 1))
 (segment (start 177.34 55.9) (end 177.34 54.2361) (width 1) (layer F.Cu) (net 1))
 (segment (start 170.6034 80.4766) (end 164.7 86.38) (width 1) (layer B.Cu) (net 1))
 (segment (start 170.6034 62.6366) (end 170.6034 80.4766) (width 1) (layer B.Cu) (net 1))
 (segment (start 177.34 55.9) (end 170.6034 62.6366) (width 1) (layer B.Cu) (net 1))
 (segment (start 178.8565 59.9565) (end 177.34 58.44) (width 0.4) (layer F.Cu) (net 2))
 (segment (start 178.8565 65.0996) (end 178.8565 59.9565) (width 0.4) (layer F.Cu) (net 2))
 (segment (start 176.7565 67.1996) (end 178.8565 65.0996) (width 0.4) (layer F.Cu) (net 2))
 (segment (start 150.8604 67.1996) (end 176.7565 67.1996) (width 0.4) (layer F.Cu) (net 2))
 (segment (start 141.84 76.22) (end 150.8604 67.1996) (width 0.4) (layer F.Cu) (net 2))
 (segment (start 131.4526 81.3) (end 141.84 81.3) (width 0.4) (layer B.Cu) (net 9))
 (segment (start 119.9612 92.7914) (end 131.4526 81.3) (width 0.4) (layer B.Cu) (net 9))
 (segment (start 108.8205 92.7914) (end 119.9612 92.7914) (width 0.4) (layer B.Cu) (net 9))
 (segment (start 105.0748 89.0457) (end 108.8205 92.7914) (width 0.4) (layer B.Cu) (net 9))
 (segment (start 105.0748 81.7382) (end 105.0748 89.0457) (width 0.4) (layer B.Cu) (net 9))
 (segment (start 95.7369 72.4003) (end 105.0748 81.7382) (width 0.4) (layer B.Cu) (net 9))
 (segment (start 94.6211 72.4003) (end 95.7369 72.4003) (width 0.4) (layer B.Cu) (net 9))
 (segment (start 93.8664 71.6456) (end 94.6211 72.4003) (width 0.4) (layer B.Cu) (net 9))
 (segment (start 93.8664 68.0361) (end 93.8664 71.6456) (width 0.4) (layer B.Cu) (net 9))
 (segment (start 94.5821 67.3204) (end 93.8664 68.0361) (width 0.4) (layer B.Cu) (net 9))
 (segment (start 95.6924 67.3204) (end 94.5821 67.3204) (width 0.4) (layer B.Cu) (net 9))
 (segment (start 96.4216 66.5912) (end 95.6924 67.3204) (width 0.4) (layer B.Cu) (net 9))
 (segment (start 96.4216 64.7956) (end 96.4216 66.5912) (width 0.4) (layer B.Cu) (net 9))
 (segment (start 95.144 63.518) (end 96.4216 64.7956) (width 0.4) (layer B.Cu) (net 9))
 (segment (start 166.1562 82.3838) (end 164.7 83.84) (width 0.4) (layer B.Cu) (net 11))
 (segment (start 166.1562 52.6502) (end 166.1562 82.3838) (width 0.4) (layer B.Cu) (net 11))
 (segment (start 164.5648 51.0588) (end 166.1562 52.6502) (width 0.4) (layer B.Cu) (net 11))
 (segment (start 102.5232 51.0588) (end 164.5648 51.0588) (width 0.4) (layer B.Cu) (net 11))
 (segment (start 95.144 58.438) (end 102.5232 51.0588) (width 0.4) (layer B.Cu) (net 11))
 (via (at 150.5143 83.5362) (size 0.6) (layers F.Cu B.Cu) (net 12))
 (segment (start 152.7505 81.3) (end 150.5143 83.5362) (width 0.4) (layer F.Cu) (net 12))
 (segment (start 164.7 81.3) (end 152.7505 81.3) (width 0.4) (layer F.Cu) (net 12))
 (segment (start 140.5588 93.4917) (end 150.5143 83.5362) (width 0.4) (layer B.Cu) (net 12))
 (segment (start 108.5305 93.4917) (end 140.5588 93.4917) (width 0.4) (layer B.Cu) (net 12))
 (segment (start 104.1268 89.088) (end 108.5305 93.4917) (width 0.4) (layer B.Cu) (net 12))
 (segment (start 104.1268 83.3766) (end 104.1268 89.088) (width 0.4) (layer B.Cu) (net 12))
 (segment (start 95.6982 74.948) (end 104.1268 83.3766) (width 0.4) (layer B.Cu) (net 12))
 (segment (start 94.5628 74.948) (end 95.6982 74.948) (width 0.4) (layer B.Cu) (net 12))
 (segment (start 93.1661 73.5513) (end 94.5628 74.948) (width 0.4) (layer B.Cu) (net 12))
 (segment (start 93.1661 67.6645) (end 93.1661 73.5513) (width 0.4) (layer B.Cu) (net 12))
 (segment (start 94.7726 66.058) (end 93.1661 67.6645) (width 0.4) (layer B.Cu) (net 12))
 (segment (start 95.144 66.058) (end 94.7726 66.058) (width 0.4) (layer B.Cu) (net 12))
 (via (at 129.4432 65.1114) (size 0.6) (layers F.Cu B.Cu) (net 14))
 (via (at 149.5079 67.2688) (size 0.6) (layers F.Cu B.Cu) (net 14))
 (segment (start 155.7488 67.2688) (end 149.5079 67.2688) (width 0.4) (layer B.Cu) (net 14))
 (segment (start 164.7 76.22) (end 155.7488 67.2688) (width 0.4) (layer B.Cu) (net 14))
 (segment (start 124.1537 70.4009) (end 129.4432 65.1114) (width 0.4) (layer B.Cu) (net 14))
 (segment (start 106.6967 70.4009) (end 124.1537 70.4009) (width 0.4) (layer B.Cu) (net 14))
 (segment (start 104.6038 68.308) (end 106.6967 70.4009) (width 0.4) (layer B.Cu) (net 14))
 (segment (start 95.434 68.308) (end 104.6038 68.308) (width 0.4) (layer B.Cu) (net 14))
 (segment (start 95.144 68.598) (end 95.434 68.308) (width 0.4) (layer B.Cu) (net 14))
 (segment (start 130.6183 66.2865) (end 129.4432 65.1114) (width 0.4) (layer F.Cu) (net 14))
 (segment (start 142.048 66.2865) (end 130.6183 66.2865) (width 0.4) (layer F.Cu) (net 14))
 (segment (start 143.0303 67.2688) (end 142.048 66.2865) (width 0.4) (layer F.Cu) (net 14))
 (segment (start 149.5079 67.2688) (end 143.0303 67.2688) (width 0.4) (layer F.Cu) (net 14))
 (segment (start 117.475 58.674) (end 112.649 63.5) (width 1) (layer F.Cu) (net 26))
 (segment (start 116.92 58.119) (end 116.92 53.58) (width 1) (layer F.Cu) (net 26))
 (segment (start 117.475 58.674) (end 116.92 58.119) (width 1) (layer F.Cu) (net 26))
 (segment (start 137.84 57.565) (end 134.908 60.497) (width 1.5) (layer B.Cu) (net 19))
 (segment (start 137.84 53.58) (end 137.84 57.565) (width 1.5) (layer B.Cu) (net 19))
 (via (at 132.0435 61.9525) (size 0.6) (layers F.Cu B.Cu) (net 20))
 (segment (start 132.76 53.58) (end 132.76 56.6303) (width 1.5) (layer B.Cu) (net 20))
 (segment (start 132.0435 57.3468) (end 132.0435 61.9525) (width 1.5) (layer B.Cu) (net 20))
 (segment (start 132.76 56.6303) (end 132.0435 57.3468) (width 1.5) (layer B.Cu) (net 20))
 (segment (start 132.0435 61.9525) (end 134.908 64.817) (width 1.5) (layer F.Cu) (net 20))
 (segment (start 107.818 63.505) (end 107.818 63.592) (width 0.4) (layer F.Cu) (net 18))
 (segment (start 112.649 58.674) (end 107.818 63.505) (width 0.4) (layer F.Cu) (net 18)))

